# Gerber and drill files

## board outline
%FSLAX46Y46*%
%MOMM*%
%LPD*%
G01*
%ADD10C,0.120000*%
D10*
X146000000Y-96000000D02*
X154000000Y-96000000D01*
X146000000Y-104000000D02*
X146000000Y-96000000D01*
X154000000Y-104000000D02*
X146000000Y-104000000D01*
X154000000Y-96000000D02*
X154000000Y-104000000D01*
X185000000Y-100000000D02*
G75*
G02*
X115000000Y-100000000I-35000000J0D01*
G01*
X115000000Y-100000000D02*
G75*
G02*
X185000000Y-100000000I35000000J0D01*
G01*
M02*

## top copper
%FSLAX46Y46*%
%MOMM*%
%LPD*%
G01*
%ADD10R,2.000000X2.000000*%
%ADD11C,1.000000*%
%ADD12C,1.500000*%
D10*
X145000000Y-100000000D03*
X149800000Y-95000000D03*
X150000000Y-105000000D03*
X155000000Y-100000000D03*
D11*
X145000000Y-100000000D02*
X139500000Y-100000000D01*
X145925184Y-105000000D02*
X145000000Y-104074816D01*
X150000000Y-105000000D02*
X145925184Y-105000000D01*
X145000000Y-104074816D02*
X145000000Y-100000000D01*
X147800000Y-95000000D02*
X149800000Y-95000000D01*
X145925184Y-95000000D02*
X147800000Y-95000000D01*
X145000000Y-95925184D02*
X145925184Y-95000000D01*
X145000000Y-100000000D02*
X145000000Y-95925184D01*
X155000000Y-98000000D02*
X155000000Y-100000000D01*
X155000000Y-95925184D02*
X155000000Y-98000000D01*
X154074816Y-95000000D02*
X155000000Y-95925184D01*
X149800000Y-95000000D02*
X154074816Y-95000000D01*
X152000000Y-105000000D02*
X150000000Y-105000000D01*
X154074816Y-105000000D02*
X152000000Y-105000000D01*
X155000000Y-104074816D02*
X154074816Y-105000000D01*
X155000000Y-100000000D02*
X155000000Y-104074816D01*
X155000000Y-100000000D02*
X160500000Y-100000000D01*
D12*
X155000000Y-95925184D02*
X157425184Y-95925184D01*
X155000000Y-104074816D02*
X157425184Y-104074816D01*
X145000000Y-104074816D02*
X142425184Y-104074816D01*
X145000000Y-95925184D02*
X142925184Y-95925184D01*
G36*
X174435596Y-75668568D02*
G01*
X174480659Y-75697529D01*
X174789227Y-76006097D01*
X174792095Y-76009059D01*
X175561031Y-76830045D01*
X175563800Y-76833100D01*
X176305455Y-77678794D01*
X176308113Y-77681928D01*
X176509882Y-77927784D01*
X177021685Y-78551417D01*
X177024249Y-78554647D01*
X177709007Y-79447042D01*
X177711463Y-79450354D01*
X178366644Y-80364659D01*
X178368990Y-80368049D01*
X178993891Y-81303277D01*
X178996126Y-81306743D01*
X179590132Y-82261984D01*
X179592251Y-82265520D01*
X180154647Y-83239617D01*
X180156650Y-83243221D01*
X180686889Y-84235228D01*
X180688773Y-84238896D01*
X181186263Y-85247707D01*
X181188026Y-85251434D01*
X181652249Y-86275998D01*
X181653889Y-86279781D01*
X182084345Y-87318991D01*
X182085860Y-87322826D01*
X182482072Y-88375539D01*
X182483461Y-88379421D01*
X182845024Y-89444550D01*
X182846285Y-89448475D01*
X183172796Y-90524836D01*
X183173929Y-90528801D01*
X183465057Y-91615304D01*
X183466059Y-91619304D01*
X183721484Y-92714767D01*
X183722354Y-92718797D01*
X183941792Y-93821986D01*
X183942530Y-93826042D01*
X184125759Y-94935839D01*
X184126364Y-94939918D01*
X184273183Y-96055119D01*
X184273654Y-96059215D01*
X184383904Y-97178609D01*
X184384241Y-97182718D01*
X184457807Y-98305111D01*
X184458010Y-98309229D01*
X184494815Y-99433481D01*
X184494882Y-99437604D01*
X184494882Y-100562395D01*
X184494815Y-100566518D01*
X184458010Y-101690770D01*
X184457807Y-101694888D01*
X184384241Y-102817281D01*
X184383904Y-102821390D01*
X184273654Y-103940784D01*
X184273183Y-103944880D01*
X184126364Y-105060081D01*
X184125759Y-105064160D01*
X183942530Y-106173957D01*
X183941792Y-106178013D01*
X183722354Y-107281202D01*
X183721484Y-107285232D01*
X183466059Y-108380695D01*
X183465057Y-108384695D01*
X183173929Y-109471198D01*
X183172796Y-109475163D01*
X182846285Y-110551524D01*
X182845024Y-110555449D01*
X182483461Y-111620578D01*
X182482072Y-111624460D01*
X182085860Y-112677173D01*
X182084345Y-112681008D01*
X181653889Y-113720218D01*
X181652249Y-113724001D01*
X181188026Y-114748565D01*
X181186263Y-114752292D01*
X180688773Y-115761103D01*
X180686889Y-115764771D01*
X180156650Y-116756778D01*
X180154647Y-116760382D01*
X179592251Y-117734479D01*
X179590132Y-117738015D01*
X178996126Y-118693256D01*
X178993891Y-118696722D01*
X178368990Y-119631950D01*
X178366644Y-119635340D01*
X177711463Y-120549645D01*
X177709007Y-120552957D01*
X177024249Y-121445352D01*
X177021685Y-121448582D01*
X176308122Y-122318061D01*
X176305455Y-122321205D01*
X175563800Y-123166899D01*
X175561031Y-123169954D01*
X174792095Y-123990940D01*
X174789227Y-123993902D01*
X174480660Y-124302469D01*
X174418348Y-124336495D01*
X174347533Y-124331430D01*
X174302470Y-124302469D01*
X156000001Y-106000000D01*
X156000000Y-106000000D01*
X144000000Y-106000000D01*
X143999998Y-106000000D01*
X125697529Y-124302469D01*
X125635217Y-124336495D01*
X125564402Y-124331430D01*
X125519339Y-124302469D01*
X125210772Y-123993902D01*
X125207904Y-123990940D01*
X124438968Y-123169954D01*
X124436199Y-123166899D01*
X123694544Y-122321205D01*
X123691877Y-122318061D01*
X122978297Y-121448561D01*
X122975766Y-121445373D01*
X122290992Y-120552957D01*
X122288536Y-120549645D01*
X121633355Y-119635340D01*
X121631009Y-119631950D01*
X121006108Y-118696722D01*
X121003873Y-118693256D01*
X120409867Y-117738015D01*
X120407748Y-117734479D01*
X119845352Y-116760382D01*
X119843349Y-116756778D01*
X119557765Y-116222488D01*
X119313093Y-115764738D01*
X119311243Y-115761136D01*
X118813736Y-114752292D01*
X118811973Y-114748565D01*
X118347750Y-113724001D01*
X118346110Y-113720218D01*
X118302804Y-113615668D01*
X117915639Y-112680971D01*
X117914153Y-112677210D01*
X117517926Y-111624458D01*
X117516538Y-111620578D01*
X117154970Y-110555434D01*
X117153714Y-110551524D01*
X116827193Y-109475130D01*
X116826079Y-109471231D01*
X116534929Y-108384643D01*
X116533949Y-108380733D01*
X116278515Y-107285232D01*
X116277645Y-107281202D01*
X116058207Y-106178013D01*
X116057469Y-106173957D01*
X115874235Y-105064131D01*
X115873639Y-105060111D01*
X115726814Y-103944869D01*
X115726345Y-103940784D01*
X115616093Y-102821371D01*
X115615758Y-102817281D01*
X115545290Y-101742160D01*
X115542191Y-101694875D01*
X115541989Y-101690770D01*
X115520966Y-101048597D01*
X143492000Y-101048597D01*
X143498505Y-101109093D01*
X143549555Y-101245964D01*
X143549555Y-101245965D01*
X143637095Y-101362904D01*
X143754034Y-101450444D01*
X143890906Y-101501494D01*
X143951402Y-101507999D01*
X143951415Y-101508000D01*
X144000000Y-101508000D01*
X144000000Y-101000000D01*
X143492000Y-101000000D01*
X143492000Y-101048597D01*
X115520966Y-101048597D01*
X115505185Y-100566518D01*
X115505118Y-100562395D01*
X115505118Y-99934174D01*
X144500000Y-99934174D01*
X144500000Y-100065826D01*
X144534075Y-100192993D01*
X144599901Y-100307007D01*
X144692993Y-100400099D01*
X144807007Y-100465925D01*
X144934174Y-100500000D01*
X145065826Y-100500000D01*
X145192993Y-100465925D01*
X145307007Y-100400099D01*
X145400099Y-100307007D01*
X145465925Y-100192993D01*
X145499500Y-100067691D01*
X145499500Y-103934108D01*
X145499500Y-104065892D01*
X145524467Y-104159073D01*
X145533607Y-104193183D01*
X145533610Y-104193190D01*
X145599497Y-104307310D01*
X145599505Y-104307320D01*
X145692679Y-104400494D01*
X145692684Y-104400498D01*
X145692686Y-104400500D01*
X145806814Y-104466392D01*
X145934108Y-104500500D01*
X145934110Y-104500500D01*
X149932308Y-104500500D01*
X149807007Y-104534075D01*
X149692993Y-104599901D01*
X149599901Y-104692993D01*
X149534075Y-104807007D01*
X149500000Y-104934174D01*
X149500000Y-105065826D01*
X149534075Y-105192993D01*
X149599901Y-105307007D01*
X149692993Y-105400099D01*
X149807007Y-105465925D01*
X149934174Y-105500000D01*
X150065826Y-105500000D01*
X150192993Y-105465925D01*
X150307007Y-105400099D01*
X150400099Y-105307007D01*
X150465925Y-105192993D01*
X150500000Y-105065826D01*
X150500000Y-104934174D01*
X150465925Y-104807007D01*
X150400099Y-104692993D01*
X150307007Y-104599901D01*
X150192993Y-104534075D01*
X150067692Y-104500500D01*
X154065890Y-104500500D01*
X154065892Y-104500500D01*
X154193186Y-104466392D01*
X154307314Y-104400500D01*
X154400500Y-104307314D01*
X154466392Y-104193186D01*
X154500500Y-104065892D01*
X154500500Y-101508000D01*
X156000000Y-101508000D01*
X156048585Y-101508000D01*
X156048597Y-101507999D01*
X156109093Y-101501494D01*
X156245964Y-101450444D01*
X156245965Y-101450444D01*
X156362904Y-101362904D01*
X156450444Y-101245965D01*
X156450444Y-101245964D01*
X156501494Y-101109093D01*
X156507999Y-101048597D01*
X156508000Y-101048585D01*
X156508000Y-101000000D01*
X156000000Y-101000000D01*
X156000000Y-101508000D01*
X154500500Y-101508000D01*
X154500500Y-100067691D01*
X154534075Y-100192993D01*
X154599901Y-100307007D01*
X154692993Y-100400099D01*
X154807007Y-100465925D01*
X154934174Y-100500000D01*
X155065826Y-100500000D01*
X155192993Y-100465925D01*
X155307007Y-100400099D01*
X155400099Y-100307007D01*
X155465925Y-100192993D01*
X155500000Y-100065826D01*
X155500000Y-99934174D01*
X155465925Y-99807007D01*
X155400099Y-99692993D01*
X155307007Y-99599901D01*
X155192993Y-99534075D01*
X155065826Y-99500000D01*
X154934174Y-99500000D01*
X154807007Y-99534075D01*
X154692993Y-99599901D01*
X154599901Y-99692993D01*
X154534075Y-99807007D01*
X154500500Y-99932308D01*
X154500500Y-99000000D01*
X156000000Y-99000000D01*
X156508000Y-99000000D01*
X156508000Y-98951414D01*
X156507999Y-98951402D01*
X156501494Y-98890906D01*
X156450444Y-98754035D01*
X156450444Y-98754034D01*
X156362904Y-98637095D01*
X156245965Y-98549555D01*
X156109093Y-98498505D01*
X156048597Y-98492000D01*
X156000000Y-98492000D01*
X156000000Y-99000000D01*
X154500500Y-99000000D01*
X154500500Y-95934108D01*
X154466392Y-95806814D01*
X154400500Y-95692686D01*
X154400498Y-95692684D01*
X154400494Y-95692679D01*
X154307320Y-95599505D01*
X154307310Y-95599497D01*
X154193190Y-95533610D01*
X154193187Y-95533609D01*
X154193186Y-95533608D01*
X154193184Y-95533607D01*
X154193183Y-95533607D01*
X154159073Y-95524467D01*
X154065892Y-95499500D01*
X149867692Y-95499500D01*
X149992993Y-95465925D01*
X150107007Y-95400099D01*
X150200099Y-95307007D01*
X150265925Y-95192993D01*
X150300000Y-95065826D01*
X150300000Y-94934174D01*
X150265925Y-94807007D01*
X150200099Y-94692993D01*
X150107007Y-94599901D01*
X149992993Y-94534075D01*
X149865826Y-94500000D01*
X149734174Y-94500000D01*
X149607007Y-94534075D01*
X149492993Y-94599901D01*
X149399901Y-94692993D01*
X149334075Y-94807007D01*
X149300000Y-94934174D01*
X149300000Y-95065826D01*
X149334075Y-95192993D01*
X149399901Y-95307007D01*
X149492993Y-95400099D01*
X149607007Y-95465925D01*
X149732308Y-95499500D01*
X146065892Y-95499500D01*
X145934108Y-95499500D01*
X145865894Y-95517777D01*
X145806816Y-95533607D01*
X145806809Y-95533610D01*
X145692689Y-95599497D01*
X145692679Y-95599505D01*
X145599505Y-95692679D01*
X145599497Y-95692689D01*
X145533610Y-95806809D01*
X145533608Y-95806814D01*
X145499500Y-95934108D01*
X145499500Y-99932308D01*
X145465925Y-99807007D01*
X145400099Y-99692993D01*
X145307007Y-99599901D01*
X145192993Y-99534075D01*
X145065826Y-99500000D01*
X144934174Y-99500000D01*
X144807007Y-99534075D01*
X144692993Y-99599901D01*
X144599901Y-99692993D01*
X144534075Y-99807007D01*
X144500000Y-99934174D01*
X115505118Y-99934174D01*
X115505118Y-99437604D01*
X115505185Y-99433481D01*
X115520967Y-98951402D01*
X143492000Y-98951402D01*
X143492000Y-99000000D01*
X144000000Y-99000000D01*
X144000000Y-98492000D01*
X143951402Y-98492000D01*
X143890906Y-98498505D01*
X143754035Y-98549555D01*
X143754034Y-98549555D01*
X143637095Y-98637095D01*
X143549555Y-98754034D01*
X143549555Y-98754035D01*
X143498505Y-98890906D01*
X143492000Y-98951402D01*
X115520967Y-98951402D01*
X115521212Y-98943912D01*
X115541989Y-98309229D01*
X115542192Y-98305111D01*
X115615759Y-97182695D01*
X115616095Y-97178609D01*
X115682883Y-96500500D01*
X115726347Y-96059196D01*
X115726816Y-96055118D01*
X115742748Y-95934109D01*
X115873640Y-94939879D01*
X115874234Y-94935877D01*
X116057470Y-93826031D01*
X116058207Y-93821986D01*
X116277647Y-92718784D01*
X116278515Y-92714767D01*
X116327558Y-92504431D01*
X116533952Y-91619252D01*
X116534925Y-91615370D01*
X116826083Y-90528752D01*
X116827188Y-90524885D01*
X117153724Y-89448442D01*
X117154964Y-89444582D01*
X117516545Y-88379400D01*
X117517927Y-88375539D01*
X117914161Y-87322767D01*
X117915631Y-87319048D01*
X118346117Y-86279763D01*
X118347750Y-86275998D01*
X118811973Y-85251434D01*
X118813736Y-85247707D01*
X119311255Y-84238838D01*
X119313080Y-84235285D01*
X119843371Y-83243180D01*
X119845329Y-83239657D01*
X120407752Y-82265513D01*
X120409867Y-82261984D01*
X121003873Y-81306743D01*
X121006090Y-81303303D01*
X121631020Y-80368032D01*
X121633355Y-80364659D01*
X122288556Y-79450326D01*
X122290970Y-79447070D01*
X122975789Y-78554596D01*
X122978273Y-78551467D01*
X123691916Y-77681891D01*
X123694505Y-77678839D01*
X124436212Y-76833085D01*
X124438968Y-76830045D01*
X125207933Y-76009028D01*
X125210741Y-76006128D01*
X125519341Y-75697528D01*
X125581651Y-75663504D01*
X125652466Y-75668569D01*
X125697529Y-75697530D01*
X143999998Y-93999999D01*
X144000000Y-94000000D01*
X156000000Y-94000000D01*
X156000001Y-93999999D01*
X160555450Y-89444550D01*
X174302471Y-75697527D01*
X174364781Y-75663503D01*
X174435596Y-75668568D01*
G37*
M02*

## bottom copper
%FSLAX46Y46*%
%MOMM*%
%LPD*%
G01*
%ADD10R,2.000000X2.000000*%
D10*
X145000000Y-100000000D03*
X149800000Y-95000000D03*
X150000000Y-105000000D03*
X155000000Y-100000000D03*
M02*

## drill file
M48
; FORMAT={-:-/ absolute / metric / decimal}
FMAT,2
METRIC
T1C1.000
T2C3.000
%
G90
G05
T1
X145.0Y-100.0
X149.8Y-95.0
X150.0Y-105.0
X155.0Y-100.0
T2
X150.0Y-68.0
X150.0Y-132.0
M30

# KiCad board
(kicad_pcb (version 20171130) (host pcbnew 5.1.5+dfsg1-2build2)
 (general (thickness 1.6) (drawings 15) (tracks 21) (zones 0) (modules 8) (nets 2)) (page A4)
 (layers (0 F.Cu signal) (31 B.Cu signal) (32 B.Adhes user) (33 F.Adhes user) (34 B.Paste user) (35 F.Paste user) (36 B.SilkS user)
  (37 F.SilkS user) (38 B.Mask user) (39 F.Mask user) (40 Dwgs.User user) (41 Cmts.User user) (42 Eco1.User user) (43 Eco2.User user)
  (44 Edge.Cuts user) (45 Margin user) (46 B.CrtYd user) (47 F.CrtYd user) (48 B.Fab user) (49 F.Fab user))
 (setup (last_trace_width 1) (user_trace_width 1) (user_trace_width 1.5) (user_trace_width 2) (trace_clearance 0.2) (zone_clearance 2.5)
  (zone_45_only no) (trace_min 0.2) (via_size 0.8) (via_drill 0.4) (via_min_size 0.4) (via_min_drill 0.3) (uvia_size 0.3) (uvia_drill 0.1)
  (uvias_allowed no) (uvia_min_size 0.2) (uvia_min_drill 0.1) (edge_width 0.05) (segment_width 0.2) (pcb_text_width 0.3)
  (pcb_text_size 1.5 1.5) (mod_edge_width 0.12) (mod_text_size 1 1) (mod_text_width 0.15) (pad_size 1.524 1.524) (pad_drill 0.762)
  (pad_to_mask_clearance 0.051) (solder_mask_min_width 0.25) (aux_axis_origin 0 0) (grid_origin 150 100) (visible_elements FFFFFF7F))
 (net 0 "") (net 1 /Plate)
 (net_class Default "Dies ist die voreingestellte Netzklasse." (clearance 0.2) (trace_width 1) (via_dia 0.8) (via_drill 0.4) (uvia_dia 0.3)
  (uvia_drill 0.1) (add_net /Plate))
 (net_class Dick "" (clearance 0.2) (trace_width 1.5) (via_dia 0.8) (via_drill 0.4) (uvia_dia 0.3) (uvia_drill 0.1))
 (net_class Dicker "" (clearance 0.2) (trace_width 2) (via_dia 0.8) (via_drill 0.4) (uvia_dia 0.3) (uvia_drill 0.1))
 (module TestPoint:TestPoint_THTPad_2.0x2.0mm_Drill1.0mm (layer F.Cu) (at 145 100)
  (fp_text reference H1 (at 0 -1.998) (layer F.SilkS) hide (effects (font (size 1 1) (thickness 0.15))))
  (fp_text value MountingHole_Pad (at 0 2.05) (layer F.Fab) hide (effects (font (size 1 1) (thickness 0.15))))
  (pad 1 thru_hole rect (at 0 0) (size 2 2) (drill 1) (layers *.Cu *.Mask) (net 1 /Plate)))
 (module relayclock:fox (layer F.Cu) (at 157 126)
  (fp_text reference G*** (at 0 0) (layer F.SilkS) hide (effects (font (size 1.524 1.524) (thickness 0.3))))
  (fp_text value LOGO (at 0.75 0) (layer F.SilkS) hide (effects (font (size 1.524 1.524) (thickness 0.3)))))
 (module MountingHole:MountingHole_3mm (layer F.Cu) (at 150 132)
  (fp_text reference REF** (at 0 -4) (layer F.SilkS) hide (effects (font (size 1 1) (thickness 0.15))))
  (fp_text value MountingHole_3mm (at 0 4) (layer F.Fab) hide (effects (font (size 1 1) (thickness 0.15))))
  (pad 1 np_thru_hole circle (at 0 0) (size 3 3) (drill 3) (layers *.Cu *.Mask)))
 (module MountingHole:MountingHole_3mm (layer F.Cu) (at 150 68)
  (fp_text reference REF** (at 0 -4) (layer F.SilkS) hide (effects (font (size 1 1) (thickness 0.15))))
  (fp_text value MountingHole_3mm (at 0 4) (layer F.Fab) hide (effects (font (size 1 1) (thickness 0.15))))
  (pad 1 np_thru_hole circle (at 0 0) (size 3 3) (drill 3) (layers *.Cu *.Mask)))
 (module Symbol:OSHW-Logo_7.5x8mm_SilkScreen (layer F.Cu) (at 144 123)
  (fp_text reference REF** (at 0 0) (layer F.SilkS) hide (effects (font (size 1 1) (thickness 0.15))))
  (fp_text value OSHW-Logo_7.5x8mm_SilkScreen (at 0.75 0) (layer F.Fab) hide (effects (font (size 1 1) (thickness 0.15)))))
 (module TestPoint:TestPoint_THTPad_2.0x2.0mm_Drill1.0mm (layer F.Cu) (at 149.8 95)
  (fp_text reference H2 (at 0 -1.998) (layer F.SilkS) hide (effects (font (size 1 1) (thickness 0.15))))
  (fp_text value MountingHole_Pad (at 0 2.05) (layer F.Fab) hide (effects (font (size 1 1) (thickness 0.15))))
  (pad 1 thru_hole rect (at 0 0) (size 2 2) (drill 1) (layers *.Cu *.Mask) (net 1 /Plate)))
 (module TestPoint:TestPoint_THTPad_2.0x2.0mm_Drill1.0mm (layer F.Cu) (at 150 105 180)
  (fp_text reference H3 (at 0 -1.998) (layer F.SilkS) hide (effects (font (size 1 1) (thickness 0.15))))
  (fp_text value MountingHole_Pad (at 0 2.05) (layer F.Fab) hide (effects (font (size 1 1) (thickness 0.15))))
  (pad 1 thru_hole rect (at 0 0 180) (size 2 2) (drill 1) (layers *.Cu *.Mask) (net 1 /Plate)))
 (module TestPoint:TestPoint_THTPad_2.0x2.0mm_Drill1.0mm (layer F.Cu) (at 155 100)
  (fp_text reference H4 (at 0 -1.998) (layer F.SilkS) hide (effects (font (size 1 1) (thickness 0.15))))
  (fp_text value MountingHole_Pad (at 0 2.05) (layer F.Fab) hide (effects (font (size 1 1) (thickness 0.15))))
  (pad 1 thru_hole rect (at 0 0) (size 2 2) (drill 1) (layers *.Cu *.Mask) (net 1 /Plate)))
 (gr_line (start 146 96) (end 154 96) (layer Edge.Cuts) (width 0.12))
 (gr_line (start 146 104) (end 146 96) (layer Edge.Cuts) (width 0.12))
 (gr_line (start 154 104) (end 146 104) (layer Edge.Cuts) (width 0.12))
 (gr_line (start 154 96) (end 154 104) (layer Edge.Cuts) (width 0.12))
 (gr_circle (center 150 100) (end 185 100) (layer Edge.Cuts) (width 0.12))
 (segment (start 145 100) (end 139.5 100) (width 1) (layer F.Cu) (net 1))
 (segment (start 145.925184 105) (end 145 104.074816) (width 1) (layer F.Cu) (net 1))
 (segment (start 150 105) (end 145.925184 105) (width 1) (layer F.Cu) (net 1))
 (segment (start 145 104.074816) (end 145 100) (width 1) (layer F.Cu) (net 1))
 (segment (start 147.8 95) (end 149.8 95) (width 1) (layer F.Cu) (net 1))
 (segment (start 145.925184 95) (end 147.8 95) (width 1) (layer F.Cu) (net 1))
 (segment (start 145 95.925184) (end 145.925184 95) (width 1) (layer F.Cu) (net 1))
 (segment (start 145 100) (end 145 95.925184) (width 1) (layer F.Cu) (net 1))
 (segment (start 155 98) (end 155 100) (width 1) (layer F.Cu) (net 1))
 (segment (start 155 95.925184) (end 155 98) (width 1) (layer F.Cu) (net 1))
 (segment (start 154.074816 95) (end 155 95.925184) (width 1) (layer F.Cu) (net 1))
 (segment (start 149.8 95) (end 154.074816 95) (width 1) (layer F.Cu) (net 1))
 (segment (start 152 105) (end 150 105) (width 1) (layer F.Cu) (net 1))
 (segment (start 154.074816 105) (end 152 105) (width 1) (layer F.Cu) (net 1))
 (segment (start 155 104.074816) (end 154.074816 105) (width 1) (layer F.Cu) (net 1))
 (segment (start 155 100) (end 155 104.074816) (width 1) (layer F.Cu) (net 1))
 (segment (start 155 100) (end 160.5 100) (width 1) (layer F.Cu) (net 1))
 (segment (start 155 95.925184) (end 157.425184 95.925184) (width 1.5) (layer F.Cu) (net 1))
 (segment (start 155 104.074816) (end 157.425184 104.074816) (width 1.5) (layer F.Cu) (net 1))
 (segment (start 145 104.074816) (end 142.425184 104.074816) (width 1.5) (layer F.Cu) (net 1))
 (segment (start 145 95.925184) (end 142.925184 95.925184) (width 1.5) (layer F.Cu) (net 1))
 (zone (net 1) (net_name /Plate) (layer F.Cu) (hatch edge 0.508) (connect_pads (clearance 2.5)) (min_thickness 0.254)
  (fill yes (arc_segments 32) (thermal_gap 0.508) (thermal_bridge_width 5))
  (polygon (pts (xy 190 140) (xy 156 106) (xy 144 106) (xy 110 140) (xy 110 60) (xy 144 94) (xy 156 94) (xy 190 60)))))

